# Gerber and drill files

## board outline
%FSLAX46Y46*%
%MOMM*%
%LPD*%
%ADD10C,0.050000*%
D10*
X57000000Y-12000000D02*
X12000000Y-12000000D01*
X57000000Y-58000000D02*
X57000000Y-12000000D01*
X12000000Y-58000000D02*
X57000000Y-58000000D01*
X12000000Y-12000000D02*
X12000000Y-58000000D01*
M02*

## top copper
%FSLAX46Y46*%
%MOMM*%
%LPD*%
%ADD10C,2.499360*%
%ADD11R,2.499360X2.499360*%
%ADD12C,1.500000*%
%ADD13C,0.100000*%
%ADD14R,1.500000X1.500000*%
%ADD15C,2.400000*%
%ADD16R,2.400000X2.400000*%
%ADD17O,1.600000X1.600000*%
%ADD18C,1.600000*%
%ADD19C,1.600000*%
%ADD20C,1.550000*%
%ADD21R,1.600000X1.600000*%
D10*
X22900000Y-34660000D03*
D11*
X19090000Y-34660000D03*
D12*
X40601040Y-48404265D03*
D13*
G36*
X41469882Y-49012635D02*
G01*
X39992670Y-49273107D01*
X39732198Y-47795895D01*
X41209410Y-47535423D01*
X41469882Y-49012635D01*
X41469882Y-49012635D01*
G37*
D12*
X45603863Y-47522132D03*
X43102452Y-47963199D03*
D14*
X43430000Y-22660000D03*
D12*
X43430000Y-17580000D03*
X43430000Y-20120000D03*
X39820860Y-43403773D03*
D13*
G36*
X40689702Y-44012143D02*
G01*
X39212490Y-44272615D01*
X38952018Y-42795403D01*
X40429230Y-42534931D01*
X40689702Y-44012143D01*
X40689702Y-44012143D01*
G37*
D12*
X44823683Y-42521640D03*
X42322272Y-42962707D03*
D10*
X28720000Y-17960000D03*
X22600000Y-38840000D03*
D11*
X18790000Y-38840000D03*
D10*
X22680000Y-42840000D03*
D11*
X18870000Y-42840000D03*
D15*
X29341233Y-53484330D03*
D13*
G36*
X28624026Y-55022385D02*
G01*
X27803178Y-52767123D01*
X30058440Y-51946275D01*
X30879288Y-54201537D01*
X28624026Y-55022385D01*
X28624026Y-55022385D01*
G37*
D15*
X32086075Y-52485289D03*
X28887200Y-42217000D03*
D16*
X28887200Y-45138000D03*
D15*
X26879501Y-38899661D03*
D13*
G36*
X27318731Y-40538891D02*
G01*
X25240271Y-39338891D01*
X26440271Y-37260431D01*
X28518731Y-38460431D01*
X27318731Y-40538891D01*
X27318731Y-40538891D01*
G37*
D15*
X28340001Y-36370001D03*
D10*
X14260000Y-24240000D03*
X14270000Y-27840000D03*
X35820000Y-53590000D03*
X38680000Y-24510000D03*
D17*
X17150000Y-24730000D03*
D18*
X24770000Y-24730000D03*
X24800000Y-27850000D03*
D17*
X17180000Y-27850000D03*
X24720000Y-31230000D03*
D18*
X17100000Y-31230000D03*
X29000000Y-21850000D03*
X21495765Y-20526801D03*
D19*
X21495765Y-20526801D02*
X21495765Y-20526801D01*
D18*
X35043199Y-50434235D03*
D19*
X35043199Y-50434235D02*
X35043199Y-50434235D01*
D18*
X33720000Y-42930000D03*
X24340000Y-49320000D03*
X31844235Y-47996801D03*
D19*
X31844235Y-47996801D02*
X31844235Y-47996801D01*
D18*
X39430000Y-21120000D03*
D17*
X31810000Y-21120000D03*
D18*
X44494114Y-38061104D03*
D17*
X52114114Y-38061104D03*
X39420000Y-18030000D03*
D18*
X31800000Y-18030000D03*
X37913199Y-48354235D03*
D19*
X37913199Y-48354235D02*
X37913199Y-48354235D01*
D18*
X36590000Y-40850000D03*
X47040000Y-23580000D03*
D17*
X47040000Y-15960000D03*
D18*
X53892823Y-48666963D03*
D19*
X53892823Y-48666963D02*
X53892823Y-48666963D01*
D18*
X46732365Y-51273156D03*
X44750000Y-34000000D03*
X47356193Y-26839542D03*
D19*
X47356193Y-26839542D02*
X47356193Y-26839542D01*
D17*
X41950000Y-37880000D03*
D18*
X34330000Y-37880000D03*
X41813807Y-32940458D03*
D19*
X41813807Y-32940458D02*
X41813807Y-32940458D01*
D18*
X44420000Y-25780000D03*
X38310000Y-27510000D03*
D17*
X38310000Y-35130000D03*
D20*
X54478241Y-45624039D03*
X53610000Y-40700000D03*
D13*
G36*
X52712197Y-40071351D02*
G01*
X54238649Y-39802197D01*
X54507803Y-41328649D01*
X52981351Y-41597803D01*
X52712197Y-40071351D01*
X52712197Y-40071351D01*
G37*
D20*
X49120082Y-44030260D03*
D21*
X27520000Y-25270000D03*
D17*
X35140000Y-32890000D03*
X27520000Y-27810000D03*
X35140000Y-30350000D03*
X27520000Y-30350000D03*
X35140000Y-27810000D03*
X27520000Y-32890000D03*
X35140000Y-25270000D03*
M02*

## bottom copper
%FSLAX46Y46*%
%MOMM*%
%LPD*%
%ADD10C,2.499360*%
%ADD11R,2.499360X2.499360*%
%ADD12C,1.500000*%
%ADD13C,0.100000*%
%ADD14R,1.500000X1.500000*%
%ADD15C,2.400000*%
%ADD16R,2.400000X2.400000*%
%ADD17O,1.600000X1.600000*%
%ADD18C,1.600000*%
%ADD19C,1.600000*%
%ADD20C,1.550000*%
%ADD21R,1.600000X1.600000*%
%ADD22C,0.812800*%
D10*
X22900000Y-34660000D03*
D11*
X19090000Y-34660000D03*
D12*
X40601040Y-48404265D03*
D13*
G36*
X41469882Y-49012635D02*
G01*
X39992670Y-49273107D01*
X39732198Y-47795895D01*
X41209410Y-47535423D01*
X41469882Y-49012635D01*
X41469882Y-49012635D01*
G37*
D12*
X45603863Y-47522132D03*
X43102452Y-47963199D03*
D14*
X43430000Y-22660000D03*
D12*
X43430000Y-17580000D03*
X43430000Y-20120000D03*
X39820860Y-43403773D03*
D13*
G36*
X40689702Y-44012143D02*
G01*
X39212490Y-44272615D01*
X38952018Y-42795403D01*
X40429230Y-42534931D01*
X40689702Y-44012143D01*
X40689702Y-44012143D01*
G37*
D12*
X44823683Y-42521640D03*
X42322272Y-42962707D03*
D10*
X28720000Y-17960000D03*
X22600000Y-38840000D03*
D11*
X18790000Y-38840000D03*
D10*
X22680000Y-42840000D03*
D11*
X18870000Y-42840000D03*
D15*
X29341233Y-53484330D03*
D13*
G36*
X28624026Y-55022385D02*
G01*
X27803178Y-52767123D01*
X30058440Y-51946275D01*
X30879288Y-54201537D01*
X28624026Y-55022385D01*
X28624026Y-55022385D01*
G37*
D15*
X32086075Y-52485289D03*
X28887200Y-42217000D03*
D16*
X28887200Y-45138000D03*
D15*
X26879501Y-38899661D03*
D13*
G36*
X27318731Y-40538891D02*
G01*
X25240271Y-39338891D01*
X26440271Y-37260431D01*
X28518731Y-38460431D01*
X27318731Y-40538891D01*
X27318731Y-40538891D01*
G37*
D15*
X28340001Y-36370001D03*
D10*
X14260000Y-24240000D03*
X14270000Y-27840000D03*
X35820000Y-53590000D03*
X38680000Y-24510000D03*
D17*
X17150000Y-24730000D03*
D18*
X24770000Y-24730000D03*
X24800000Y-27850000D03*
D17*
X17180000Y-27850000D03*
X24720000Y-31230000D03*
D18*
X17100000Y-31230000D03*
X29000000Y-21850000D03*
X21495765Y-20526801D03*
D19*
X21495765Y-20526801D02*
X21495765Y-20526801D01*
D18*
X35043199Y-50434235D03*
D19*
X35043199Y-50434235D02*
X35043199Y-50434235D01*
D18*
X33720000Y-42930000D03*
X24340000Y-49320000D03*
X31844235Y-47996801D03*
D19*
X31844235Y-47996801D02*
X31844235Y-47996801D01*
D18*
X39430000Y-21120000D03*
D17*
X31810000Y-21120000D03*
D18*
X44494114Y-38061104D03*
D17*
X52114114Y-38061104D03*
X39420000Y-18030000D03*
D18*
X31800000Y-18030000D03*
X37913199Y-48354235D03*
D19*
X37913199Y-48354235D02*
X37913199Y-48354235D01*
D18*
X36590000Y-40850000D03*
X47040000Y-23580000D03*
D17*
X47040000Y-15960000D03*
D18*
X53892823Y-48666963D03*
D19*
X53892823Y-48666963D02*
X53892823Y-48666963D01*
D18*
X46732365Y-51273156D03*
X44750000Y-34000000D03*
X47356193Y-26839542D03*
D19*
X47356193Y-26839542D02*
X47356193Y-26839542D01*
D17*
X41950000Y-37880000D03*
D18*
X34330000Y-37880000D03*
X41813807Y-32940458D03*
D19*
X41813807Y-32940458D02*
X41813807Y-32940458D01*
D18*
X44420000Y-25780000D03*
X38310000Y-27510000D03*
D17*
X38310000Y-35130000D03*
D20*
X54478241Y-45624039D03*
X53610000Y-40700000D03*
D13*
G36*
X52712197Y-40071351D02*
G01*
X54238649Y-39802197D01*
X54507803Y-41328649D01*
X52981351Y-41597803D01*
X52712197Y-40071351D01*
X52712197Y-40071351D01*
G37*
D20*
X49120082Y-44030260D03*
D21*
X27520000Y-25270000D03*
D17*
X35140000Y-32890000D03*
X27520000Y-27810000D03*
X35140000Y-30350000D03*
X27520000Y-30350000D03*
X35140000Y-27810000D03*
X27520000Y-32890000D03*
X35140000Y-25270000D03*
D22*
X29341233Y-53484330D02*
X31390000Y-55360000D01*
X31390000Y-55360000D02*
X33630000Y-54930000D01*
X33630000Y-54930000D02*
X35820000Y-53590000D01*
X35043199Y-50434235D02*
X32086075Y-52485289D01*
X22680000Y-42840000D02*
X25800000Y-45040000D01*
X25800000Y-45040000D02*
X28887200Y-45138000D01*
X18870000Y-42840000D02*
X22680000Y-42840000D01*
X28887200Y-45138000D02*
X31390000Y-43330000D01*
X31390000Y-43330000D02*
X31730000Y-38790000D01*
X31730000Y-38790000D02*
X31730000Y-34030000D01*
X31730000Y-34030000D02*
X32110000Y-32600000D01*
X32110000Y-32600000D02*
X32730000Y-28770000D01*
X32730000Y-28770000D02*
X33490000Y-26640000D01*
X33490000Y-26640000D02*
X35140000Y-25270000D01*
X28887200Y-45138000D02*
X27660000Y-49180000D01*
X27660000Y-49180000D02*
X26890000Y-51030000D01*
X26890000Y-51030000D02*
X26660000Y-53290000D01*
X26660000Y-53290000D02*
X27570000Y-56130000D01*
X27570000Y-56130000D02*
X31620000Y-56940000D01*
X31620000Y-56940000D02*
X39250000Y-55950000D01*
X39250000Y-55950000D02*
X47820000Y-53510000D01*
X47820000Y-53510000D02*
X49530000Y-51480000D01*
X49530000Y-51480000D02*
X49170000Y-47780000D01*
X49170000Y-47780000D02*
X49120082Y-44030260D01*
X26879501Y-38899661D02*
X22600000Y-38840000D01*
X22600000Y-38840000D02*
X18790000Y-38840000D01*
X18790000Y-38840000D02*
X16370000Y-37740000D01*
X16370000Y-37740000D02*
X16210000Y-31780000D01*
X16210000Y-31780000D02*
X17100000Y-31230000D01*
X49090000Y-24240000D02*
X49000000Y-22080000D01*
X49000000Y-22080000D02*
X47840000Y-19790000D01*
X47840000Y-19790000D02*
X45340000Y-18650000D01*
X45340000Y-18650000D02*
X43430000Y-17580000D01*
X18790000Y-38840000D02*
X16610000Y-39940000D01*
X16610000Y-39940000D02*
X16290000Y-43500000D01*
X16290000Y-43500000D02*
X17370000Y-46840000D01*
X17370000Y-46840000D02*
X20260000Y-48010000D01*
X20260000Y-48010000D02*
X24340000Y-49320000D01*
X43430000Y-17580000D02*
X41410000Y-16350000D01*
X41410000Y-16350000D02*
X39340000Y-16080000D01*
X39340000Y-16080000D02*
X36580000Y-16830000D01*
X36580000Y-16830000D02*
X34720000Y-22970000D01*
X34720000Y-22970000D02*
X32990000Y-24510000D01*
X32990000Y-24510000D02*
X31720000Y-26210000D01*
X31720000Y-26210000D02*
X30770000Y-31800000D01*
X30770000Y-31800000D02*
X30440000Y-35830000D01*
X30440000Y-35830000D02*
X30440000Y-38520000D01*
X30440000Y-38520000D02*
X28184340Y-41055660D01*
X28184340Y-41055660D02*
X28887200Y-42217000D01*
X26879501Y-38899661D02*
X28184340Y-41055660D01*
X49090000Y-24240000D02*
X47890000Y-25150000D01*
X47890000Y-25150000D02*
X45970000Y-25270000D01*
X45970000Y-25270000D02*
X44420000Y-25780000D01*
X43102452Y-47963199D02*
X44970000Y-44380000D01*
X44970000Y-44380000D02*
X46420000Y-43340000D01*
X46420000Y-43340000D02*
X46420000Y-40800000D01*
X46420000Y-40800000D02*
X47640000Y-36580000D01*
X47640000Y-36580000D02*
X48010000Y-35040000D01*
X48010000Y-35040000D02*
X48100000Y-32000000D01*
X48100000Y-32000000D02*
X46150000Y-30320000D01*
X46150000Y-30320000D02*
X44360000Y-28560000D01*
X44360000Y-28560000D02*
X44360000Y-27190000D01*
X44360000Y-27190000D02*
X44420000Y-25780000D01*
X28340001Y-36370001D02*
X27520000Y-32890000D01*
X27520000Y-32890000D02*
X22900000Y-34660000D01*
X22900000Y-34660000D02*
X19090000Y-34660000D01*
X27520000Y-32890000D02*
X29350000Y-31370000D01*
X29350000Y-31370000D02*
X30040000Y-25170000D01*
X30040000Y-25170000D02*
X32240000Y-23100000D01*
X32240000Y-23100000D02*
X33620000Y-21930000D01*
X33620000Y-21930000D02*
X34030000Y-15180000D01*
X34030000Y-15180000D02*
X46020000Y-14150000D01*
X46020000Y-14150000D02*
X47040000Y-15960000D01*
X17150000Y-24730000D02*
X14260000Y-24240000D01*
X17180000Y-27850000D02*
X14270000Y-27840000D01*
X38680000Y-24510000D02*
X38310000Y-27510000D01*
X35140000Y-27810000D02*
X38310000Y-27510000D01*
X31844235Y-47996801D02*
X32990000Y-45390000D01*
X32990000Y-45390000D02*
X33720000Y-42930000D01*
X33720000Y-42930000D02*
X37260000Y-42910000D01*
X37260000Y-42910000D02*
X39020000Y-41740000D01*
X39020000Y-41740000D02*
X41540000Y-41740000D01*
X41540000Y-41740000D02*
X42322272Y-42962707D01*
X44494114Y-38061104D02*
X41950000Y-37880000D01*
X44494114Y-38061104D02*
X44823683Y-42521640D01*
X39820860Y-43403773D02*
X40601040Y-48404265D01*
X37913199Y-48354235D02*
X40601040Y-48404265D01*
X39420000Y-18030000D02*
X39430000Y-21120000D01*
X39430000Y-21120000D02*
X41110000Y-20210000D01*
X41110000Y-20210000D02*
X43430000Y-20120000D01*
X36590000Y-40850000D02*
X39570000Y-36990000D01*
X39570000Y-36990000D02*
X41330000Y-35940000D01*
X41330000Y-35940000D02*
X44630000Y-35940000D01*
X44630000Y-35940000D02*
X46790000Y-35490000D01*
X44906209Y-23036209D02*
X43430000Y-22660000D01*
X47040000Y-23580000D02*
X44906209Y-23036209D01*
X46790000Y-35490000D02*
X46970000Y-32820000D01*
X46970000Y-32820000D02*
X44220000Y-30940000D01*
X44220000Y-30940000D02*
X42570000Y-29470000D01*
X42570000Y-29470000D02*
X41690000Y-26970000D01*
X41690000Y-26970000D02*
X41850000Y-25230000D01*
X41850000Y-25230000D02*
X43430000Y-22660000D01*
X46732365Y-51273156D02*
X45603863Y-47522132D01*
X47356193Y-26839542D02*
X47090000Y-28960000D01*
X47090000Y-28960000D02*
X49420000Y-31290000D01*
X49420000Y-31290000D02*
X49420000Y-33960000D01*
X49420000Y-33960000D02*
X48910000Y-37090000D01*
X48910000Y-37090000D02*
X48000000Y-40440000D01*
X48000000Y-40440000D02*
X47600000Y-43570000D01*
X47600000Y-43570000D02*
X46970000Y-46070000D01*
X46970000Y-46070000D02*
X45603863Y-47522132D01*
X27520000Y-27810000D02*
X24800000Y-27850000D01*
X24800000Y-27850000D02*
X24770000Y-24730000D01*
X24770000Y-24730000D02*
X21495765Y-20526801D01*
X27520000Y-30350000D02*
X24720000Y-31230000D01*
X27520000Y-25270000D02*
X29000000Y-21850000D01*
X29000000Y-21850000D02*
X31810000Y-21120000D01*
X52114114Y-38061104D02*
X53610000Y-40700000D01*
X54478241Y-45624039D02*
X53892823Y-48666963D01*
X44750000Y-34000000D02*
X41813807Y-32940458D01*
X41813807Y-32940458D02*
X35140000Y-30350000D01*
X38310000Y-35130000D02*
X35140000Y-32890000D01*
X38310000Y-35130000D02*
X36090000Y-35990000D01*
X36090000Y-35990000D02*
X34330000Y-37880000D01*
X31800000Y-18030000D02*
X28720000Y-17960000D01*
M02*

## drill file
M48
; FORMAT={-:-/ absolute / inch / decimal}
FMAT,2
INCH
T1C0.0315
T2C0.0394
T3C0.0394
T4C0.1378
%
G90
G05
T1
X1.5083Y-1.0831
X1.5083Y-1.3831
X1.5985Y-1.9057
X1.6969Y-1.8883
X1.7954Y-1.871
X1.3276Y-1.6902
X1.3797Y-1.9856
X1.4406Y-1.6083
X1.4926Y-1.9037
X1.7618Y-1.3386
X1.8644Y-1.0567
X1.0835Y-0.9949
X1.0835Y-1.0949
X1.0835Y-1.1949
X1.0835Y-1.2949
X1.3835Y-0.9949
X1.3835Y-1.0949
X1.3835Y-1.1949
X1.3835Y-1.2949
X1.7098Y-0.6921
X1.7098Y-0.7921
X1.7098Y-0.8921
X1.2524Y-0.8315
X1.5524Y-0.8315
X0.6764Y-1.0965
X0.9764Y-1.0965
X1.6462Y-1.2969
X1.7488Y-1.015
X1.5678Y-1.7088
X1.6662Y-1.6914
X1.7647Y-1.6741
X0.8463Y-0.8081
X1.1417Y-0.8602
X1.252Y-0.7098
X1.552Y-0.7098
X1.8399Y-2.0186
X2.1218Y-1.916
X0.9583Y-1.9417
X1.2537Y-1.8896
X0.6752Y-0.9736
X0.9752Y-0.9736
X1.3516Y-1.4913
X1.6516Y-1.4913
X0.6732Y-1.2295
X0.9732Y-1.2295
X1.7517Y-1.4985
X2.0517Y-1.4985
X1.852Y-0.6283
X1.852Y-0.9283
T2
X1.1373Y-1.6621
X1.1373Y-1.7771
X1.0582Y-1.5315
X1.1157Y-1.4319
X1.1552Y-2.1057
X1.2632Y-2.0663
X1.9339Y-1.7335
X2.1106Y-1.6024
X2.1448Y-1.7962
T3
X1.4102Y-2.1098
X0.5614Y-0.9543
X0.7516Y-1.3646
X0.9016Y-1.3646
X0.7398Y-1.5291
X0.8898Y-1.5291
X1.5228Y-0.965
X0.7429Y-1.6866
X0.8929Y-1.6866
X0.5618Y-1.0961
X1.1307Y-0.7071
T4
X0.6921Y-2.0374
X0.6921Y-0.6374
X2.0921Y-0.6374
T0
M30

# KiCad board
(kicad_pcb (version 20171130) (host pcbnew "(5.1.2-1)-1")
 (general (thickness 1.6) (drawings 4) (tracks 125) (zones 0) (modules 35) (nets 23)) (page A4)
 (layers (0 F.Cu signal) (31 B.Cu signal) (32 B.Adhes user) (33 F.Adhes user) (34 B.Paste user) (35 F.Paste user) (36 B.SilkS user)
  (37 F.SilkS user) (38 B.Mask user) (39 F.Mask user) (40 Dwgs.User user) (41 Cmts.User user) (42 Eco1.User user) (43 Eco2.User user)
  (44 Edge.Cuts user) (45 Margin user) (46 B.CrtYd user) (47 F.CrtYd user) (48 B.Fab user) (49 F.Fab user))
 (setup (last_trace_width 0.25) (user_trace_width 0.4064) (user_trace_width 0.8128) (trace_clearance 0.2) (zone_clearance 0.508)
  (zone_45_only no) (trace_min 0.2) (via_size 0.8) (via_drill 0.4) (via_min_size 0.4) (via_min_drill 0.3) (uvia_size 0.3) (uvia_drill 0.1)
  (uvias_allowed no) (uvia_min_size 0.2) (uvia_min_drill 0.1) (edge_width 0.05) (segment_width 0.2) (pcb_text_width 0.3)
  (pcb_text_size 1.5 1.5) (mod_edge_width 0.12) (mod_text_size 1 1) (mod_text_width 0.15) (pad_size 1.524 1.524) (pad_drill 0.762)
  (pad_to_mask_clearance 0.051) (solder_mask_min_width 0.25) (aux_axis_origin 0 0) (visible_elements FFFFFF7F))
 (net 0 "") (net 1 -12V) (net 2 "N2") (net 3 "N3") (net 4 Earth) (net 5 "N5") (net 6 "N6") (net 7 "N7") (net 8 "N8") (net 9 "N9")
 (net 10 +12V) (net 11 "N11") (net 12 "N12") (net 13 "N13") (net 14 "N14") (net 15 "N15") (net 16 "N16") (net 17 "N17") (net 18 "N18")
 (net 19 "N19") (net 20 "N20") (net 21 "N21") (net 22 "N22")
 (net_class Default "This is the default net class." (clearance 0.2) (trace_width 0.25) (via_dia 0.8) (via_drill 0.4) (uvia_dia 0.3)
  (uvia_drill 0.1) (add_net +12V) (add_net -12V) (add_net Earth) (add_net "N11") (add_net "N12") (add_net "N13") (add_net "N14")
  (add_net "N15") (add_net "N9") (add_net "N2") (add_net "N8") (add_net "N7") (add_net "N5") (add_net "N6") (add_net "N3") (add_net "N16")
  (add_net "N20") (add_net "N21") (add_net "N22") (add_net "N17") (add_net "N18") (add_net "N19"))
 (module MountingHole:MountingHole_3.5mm (layer F.Cu) (at 53.14 16.19)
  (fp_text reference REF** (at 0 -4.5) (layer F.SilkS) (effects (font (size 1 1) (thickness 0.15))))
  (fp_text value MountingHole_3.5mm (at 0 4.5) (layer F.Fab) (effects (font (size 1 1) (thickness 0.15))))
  (pad 1 np_thru_hole circle (at 0 0) (size 3.5 3.5) (drill 3.5) (layers *.Cu *.Mask)))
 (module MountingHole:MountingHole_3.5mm (layer F.Cu) (at 17.58 16.19)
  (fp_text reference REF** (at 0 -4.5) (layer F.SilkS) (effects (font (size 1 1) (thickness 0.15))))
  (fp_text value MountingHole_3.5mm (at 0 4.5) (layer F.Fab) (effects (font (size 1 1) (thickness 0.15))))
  (pad 1 np_thru_hole circle (at 0 0) (size 3.5 3.5) (drill 3.5) (layers *.Cu *.Mask)))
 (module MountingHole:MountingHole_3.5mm (layer F.Cu) (at 17.58 51.75)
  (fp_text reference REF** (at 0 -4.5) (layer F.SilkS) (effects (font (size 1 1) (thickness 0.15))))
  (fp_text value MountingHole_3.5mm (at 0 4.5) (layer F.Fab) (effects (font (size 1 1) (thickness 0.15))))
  (pad 1 np_thru_hole circle (at 0 0) (size 3.5 3.5) (drill 3.5) (layers *.Cu *.Mask)))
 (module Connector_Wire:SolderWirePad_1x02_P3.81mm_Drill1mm (layer F.Cu) (at 19.09 34.66)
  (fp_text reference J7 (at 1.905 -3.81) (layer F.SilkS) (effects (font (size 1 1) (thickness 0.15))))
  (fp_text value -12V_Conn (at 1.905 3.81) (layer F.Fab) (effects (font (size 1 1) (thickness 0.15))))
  (pad 2 thru_hole circle (at 3.81 0) (size 2.49936 2.49936) (drill 1.00076) (layers *.Cu *.Mask) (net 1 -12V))
  (pad 1 thru_hole rect (at 0 0) (size 2.49936 2.49936) (drill 1.00076) (layers *.Cu *.Mask) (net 1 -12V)))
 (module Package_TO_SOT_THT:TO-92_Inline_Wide (layer F.Cu) (at 40.60104 48.404265 10)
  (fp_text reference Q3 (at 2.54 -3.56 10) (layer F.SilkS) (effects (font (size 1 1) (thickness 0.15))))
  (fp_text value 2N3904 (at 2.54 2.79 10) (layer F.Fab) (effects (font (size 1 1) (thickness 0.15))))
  (pad 1 thru_hole rect (at 0 0 100) (size 1.5 1.5) (drill 0.8) (layers *.Cu *.Mask) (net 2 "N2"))
  (pad 3 thru_hole circle (at 5.08 0 100) (size 1.5 1.5) (drill 0.8) (layers *.Cu *.Mask) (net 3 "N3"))
  (pad 2 thru_hole circle (at 2.54 0 100) (size 1.5 1.5) (drill 0.8) (layers *.Cu *.Mask) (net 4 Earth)))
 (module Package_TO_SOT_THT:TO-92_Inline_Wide (layer F.Cu) (at 43.43 22.66 90)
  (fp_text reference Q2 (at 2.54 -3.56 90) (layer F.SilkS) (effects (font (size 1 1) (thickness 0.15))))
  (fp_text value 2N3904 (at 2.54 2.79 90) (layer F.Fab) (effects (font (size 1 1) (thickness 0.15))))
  (pad 1 thru_hole rect (at 0 0 180) (size 1.5 1.5) (drill 0.8) (layers *.Cu *.Mask) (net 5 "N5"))
  (pad 3 thru_hole circle (at 5.08 0 180) (size 1.5 1.5) (drill 0.8) (layers *.Cu *.Mask) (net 4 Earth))
  (pad 2 thru_hole circle (at 2.54 0 180) (size 1.5 1.5) (drill 0.8) (layers *.Cu *.Mask) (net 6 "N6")))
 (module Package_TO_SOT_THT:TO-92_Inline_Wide (layer F.Cu) (at 39.82086 43.403773 10)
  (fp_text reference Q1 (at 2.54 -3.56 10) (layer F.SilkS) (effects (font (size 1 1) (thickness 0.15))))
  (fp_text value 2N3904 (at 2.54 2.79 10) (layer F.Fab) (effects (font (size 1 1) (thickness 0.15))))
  (pad 1 thru_hole rect (at 0 0 100) (size 1.5 1.5) (drill 0.8) (layers *.Cu *.Mask) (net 2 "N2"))
  (pad 3 thru_hole circle (at 5.08 0 100) (size 1.5 1.5) (drill 0.8) (layers *.Cu *.Mask) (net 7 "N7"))
  (pad 2 thru_hole circle (at 2.54 0 100) (size 1.5 1.5) (drill 0.8) (layers *.Cu *.Mask) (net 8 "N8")))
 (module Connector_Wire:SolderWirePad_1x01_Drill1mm (layer F.Cu) (at 28.72 17.96)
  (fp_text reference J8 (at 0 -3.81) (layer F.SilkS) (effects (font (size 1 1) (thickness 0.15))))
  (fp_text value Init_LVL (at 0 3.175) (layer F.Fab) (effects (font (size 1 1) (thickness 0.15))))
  (pad 1 thru_hole circle (at 0 0) (size 2.49936 2.49936) (drill 1.00076) (layers *.Cu *.Mask) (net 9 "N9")))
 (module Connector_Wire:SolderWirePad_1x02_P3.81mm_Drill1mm (layer F.Cu) (at 18.79 38.84)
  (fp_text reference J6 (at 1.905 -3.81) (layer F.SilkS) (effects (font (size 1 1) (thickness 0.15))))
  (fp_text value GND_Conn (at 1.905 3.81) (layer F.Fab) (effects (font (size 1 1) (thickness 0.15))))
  (pad 2 thru_hole circle (at 3.81 0) (size 2.49936 2.49936) (drill 1.00076) (layers *.Cu *.Mask) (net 4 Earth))
  (pad 1 thru_hole rect (at 0 0) (size 2.49936 2.49936) (drill 1.00076) (layers *.Cu *.Mask) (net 4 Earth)))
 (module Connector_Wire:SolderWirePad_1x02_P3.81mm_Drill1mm (layer F.Cu) (at 18.87 42.84)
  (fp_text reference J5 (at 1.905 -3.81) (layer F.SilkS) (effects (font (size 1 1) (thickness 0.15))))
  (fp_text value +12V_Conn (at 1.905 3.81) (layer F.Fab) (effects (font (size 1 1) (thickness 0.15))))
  (pad 2 thru_hole circle (at 3.81 0) (size 2.49936 2.49936) (drill 1.00076) (layers *.Cu *.Mask) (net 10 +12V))
  (pad 1 thru_hole rect (at 0 0) (size 2.49936 2.49936) (drill 1.00076) (layers *.Cu *.Mask) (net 10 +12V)))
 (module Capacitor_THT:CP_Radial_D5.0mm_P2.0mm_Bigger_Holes (layer F.Cu) (at 31.29 53.64 20)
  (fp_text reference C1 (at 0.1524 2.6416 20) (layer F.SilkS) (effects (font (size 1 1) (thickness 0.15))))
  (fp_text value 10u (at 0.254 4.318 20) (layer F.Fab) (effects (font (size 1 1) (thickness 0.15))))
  (pad 1 thru_hole rect (at -1.778 -0.8128 20) (size 2.4 2.4) (drill 1) (layers *.Cu *.Mask) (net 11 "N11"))
  (pad 2 thru_hole circle (at 1.143 -0.8128 20) (size 2.4 2.4) (drill 1) (layers *.Cu *.Mask) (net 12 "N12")))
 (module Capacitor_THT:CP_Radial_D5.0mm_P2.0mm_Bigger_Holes (layer F.Cu) (at 29.7 43.36 90)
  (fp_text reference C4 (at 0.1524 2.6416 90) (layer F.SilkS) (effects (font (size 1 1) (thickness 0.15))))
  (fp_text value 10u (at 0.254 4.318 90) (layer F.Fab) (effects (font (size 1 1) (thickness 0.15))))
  (pad 2 thru_hole circle (at 1.143 -0.8128 90) (size 2.4 2.4) (drill 1) (layers *.Cu *.Mask) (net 4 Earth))
  (pad 1 thru_hole rect (at -1.778 -0.8128 90) (size 2.4 2.4) (drill 1) (layers *.Cu *.Mask) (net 10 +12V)))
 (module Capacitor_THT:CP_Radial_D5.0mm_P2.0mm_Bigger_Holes (layer F.Cu) (at 28.472406 37.766268 60)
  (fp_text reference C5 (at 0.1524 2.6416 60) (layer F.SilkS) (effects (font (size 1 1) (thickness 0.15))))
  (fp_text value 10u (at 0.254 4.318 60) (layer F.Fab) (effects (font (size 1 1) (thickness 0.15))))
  (pad 1 thru_hole rect (at -1.778 -0.8128 60) (size 2.4 2.4) (drill 1) (layers *.Cu *.Mask) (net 4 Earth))
  (pad 2 thru_hole circle (at 1.143 -0.8128 60) (size 2.4 2.4) (drill 1) (layers *.Cu *.Mask) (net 1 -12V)))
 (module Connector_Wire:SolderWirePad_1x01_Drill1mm (layer F.Cu) (at 14.26 24.24)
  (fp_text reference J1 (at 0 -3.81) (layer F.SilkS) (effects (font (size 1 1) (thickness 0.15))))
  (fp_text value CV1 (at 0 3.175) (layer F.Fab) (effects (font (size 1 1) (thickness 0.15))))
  (pad 1 thru_hole circle (at 0 0) (size 2.49936 2.49936) (drill 1.00076) (layers *.Cu *.Mask) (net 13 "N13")))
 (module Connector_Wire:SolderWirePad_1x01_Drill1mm (layer F.Cu) (at 14.27 27.84)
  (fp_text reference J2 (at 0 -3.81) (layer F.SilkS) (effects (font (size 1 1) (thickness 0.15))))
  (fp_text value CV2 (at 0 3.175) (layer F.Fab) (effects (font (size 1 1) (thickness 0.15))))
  (pad 1 thru_hole circle (at 0 0) (size 2.49936 2.49936) (drill 1.00076) (layers *.Cu *.Mask) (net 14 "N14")))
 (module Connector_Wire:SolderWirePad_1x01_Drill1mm (layer F.Cu) (at 35.82 53.59 10)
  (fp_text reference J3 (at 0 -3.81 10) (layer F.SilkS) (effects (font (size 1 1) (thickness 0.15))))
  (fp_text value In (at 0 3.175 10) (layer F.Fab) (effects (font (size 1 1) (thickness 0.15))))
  (pad 1 thru_hole circle (at 0 0 10) (size 2.49936 2.49936) (drill 1.00076) (layers *.Cu *.Mask) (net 11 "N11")))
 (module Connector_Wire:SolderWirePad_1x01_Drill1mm (layer F.Cu) (at 38.68 24.51)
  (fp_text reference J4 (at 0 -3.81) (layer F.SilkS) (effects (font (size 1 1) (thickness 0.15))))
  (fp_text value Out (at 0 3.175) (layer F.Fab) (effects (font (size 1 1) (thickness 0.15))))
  (pad 1 thru_hole circle (at 0 0) (size 2.49936 2.49936) (drill 1.00076) (layers *.Cu *.Mask) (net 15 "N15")))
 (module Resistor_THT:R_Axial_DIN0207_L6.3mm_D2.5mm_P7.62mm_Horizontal (layer F.Cu) (at 24.77 24.73 180)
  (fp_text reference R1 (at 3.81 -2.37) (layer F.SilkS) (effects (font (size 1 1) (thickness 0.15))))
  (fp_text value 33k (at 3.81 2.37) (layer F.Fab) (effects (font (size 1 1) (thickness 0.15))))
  (pad 2 thru_hole oval (at 7.62 0 180) (size 1.6 1.6) (drill 0.8) (layers *.Cu *.Mask) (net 13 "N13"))
  (pad 1 thru_hole circle (at 0 0 180) (size 1.6 1.6) (drill 0.8) (layers *.Cu *.Mask) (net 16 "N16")))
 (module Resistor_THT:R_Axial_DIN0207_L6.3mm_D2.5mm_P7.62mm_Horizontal (layer F.Cu) (at 24.8 27.85 180)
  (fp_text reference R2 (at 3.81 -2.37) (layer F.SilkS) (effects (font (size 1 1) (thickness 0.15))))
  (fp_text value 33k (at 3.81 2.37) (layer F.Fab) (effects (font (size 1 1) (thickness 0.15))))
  (pad 1 thru_hole circle (at 0 0 180) (size 1.6 1.6) (drill 0.8) (layers *.Cu *.Mask) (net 16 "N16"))
  (pad 2 thru_hole oval (at 7.62 0 180) (size 1.6 1.6) (drill 0.8) (layers *.Cu *.Mask) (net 14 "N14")))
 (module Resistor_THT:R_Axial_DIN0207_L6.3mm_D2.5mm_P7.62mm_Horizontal (layer F.Cu) (at 17.1 31.23)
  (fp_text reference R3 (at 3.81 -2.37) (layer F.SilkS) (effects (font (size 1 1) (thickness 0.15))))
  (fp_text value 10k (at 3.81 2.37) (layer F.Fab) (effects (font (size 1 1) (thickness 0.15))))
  (pad 2 thru_hole oval (at 7.62 0) (size 1.6 1.6) (drill 0.8) (layers *.Cu *.Mask) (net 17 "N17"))
  (pad 1 thru_hole circle (at 0 0) (size 1.6 1.6) (drill 0.8) (layers *.Cu *.Mask) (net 4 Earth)))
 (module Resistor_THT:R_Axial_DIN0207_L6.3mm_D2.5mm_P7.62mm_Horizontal (layer F.Cu) (at 29 21.85 170)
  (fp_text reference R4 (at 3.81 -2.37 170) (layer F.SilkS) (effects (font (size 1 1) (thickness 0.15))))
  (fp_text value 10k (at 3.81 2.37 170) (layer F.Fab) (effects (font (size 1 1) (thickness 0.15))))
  (pad 1 thru_hole circle (at 0 0 170) (size 1.6 1.6) (drill 0.8) (layers *.Cu *.Mask) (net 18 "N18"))
  (pad 2 thru_hole oval (at 7.62 0 170) (size 1.6 1.6) (drill 0.8) (layers *.Cu *.Mask) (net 16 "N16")))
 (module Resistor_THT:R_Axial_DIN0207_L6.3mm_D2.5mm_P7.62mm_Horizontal (layer F.Cu) (at 33.72 42.93 280)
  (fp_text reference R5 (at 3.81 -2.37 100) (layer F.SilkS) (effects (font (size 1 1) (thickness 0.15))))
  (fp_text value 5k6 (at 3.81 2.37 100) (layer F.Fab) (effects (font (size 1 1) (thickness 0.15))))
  (pad 2 thru_hole oval (at 7.62 0 280) (size 1.6 1.6) (drill 0.8) (layers *.Cu *.Mask) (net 12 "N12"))
  (pad 1 thru_hole circle (at 0 0 280) (size 1.6 1.6) (drill 0.8) (layers *.Cu *.Mask) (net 8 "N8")))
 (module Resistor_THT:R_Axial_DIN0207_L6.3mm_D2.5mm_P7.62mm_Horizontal (layer F.Cu) (at 24.34 49.32 10)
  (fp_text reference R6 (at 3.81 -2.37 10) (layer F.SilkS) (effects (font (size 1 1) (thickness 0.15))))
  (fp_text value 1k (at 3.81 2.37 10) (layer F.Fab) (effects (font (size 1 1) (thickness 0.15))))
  (pad 1 thru_hole circle (at 0 0 10) (size 1.6 1.6) (drill 0.8) (layers *.Cu *.Mask) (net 4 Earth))
  (pad 2 thru_hole oval (at 7.62 0 10) (size 1.6 1.6) (drill 0.8) (layers *.Cu *.Mask) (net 8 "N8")))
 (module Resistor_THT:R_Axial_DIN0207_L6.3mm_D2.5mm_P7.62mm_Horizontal (layer F.Cu) (at 39.43 21.12 180)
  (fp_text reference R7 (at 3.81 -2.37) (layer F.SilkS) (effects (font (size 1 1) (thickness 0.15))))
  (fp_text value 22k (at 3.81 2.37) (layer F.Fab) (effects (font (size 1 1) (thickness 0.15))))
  (pad 1 thru_hole circle (at 0 0 180) (size 1.6 1.6) (drill 0.8) (layers *.Cu *.Mask) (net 6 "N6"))
  (pad 2 thru_hole oval (at 7.62 0 180) (size 1.6 1.6) (drill 0.8) (layers *.Cu *.Mask) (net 18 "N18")))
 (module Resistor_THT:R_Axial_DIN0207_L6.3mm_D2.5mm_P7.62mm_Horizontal (layer F.Cu) (at 44.494114 38.061104)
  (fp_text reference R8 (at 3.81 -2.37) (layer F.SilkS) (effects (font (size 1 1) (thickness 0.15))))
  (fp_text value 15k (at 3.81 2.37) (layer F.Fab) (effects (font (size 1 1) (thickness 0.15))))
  (pad 1 thru_hole circle (at 0 0) (size 1.6 1.6) (drill 0.8) (layers *.Cu *.Mask) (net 7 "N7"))
  (pad 2 thru_hole oval (at 7.62 0) (size 1.6 1.6) (drill 0.8) (layers *.Cu *.Mask) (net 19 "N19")))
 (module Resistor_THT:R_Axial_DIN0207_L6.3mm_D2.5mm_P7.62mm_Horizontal (layer F.Cu) (at 31.8 18.03)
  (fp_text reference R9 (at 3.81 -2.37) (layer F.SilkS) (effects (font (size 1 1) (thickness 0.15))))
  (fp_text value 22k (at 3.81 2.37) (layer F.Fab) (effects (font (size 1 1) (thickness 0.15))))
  (pad 2 thru_hole oval (at 7.62 0) (size 1.6 1.6) (drill 0.8) (layers *.Cu *.Mask) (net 6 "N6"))
  (pad 1 thru_hole circle (at 0 0) (size 1.6 1.6) (drill 0.8) (layers *.Cu *.Mask) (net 9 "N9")))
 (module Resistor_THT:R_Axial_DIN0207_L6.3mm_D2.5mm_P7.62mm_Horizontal (layer F.Cu) (at 36.59 40.85 280)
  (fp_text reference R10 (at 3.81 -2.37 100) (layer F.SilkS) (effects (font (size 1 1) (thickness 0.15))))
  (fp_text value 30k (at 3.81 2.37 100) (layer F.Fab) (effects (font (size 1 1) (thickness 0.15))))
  (pad 2 thru_hole oval (at 7.62 0 280) (size 1.6 1.6) (drill 0.8) (layers *.Cu *.Mask) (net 2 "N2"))
  (pad 1 thru_hole circle (at 0 0 280) (size 1.6 1.6) (drill 0.8) (layers *.Cu *.Mask) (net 5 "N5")))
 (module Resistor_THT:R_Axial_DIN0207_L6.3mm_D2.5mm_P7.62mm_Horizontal (layer F.Cu) (at 47.04 23.58 90)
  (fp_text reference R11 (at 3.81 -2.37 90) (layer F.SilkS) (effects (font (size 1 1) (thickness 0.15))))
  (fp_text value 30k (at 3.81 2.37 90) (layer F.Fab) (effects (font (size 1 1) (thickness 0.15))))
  (pad 1 thru_hole circle (at 0 0 90) (size 1.6 1.6) (drill 0.8) (layers *.Cu *.Mask) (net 5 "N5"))
  (pad 2 thru_hole oval (at 7.62 0 90) (size 1.6 1.6) (drill 0.8) (layers *.Cu *.Mask) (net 1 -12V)))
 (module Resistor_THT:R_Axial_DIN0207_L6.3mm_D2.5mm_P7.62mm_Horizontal (layer F.Cu) (at 46.732365 51.273156 20)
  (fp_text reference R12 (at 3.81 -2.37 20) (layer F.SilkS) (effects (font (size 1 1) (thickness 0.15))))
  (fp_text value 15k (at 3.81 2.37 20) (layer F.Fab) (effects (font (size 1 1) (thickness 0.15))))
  (pad 2 thru_hole oval (at 7.62 0 20) (size 1.6 1.6) (drill 0.8) (layers *.Cu *.Mask) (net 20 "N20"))
  (pad 1 thru_hole circle (at 0 0 20) (size 1.6 1.6) (drill 0.8) (layers *.Cu *.Mask) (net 3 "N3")))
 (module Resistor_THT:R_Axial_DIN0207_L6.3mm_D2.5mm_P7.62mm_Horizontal (layer F.Cu) (at 44.75 34 70)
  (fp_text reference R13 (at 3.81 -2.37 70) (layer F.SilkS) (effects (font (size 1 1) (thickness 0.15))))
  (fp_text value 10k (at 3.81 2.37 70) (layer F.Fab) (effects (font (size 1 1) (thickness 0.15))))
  (pad 1 thru_hole circle (at 0 0 70) (size 1.6 1.6) (drill 0.8) (layers *.Cu *.Mask) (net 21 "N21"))
  (pad 2 thru_hole oval (at 7.62 0 70) (size 1.6 1.6) (drill 0.8) (layers *.Cu *.Mask) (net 3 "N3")))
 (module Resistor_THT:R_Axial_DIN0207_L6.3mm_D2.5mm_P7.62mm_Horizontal (layer F.Cu) (at 34.33 37.88)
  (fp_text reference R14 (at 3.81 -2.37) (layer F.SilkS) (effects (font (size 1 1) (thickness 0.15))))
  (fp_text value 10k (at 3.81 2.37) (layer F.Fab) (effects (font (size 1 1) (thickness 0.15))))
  (pad 2 thru_hole oval (at 7.62 0) (size 1.6 1.6) (drill 0.8) (layers *.Cu *.Mask) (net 7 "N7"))
  (pad 1 thru_hole circle (at 0 0) (size 1.6 1.6) (drill 0.8) (layers *.Cu *.Mask) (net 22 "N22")))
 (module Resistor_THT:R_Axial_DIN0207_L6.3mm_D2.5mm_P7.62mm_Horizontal (layer F.Cu) (at 44.42 25.78 250)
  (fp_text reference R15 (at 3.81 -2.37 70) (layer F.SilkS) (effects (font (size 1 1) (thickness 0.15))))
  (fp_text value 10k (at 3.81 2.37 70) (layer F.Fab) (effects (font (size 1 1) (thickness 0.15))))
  (pad 2 thru_hole oval (at 7.62 0 250) (size 1.6 1.6) (drill 0.8) (layers *.Cu *.Mask) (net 21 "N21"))
  (pad 1 thru_hole circle (at 0 0 250) (size 1.6 1.6) (drill 0.8) (layers *.Cu *.Mask) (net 4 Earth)))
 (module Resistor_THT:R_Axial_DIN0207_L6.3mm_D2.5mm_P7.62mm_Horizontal (layer F.Cu) (at 38.31 27.51 270)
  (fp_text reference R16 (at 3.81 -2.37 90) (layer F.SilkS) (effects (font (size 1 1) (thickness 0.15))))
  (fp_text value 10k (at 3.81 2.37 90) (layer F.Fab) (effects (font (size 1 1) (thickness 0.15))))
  (pad 1 thru_hole circle (at 0 0 270) (size 1.6 1.6) (drill 0.8) (layers *.Cu *.Mask) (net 15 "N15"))
  (pad 2 thru_hole oval (at 7.62 0 270) (size 1.6 1.6) (drill 0.8) (layers *.Cu *.Mask) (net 22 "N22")))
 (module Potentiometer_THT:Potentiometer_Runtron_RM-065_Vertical (layer F.Cu) (at 53.61 40.7 280)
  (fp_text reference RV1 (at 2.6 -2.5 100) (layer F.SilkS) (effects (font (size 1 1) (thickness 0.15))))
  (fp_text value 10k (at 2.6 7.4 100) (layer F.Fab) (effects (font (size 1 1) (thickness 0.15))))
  (pad 3 thru_hole circle (at 5 0 280) (size 1.55 1.55) (drill 1) (layers *.Cu *.Mask) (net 20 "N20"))
  (pad 1 thru_hole rect (at 0 0 280) (size 1.55 1.55) (drill 1) (layers *.Cu *.Mask) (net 19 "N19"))
  (pad 2 thru_hole circle (at 2.5 5 280) (size 1.55 1.55) (drill 1) (layers *.Cu *.Mask) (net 10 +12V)))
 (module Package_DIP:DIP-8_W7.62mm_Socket (layer F.Cu) (at 27.52 25.27)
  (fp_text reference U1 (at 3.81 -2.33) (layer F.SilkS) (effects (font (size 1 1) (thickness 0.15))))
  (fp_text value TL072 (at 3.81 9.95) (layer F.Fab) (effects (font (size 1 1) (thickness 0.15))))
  (pad 1 thru_hole rect (at 0 0) (size 1.6 1.6) (drill 0.8) (layers *.Cu *.Mask) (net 18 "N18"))
  (pad 5 thru_hole oval (at 7.62 7.62) (size 1.6 1.6) (drill 0.8) (layers *.Cu *.Mask) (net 22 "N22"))
  (pad 2 thru_hole oval (at 0 2.54) (size 1.6 1.6) (drill 0.8) (layers *.Cu *.Mask) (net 16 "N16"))
  (pad 6 thru_hole oval (at 7.62 5.08) (size 1.6 1.6) (drill 0.8) (layers *.Cu *.Mask) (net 21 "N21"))
  (pad 3 thru_hole oval (at 0 5.08) (size 1.6 1.6) (drill 0.8) (layers *.Cu *.Mask) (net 17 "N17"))
  (pad 7 thru_hole oval (at 7.62 2.54) (size 1.6 1.6) (drill 0.8) (layers *.Cu *.Mask) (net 15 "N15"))
  (pad 4 thru_hole oval (at 0 7.62) (size 1.6 1.6) (drill 0.8) (layers *.Cu *.Mask) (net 1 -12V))
  (pad 8 thru_hole oval (at 7.62 0) (size 1.6 1.6) (drill 0.8) (layers *.Cu *.Mask) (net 10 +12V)))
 (gr_line (start 57 12) (end 12 12) (layer Edge.Cuts) (width 0.05))
 (gr_line (start 57 58) (end 57 12) (layer Edge.Cuts) (width 0.05))
 (gr_line (start 12 58) (end 57 58) (layer Edge.Cuts) (width 0.05))
 (gr_line (start 12 12) (end 12 58) (layer Edge.Cuts) (width 0.05))
 (segment (start 29.341233 53.48433) (end 31.39 55.36) (width 0.8128) (layer B.Cu) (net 11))
 (segment (start 31.39 55.36) (end 33.63 54.93) (width 0.8128) (layer B.Cu) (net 11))
 (segment (start 33.63 54.93) (end 35.82 53.59) (width 0.8128) (layer B.Cu) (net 11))
 (segment (start 35.043199 50.434235) (end 32.086075 52.485289) (width 0.8128) (layer B.Cu) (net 12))
 (segment (start 22.68 42.84) (end 25.8 45.04) (width 0.8128) (layer B.Cu) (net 10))
 (segment (start 25.8 45.04) (end 28.8872 45.138) (width 0.8128) (layer B.Cu) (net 10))
 (segment (start 18.87 42.84) (end 22.68 42.84) (width 0.8128) (layer B.Cu) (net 10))
 (segment (start 28.8872 45.138) (end 31.39 43.33) (width 0.8128) (layer B.Cu) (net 10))
 (segment (start 31.39 43.33) (end 31.73 38.79) (width 0.8128) (layer B.Cu) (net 10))
 (segment (start 31.73 38.79) (end 31.73 34.03) (width 0.8128) (layer B.Cu) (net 10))
 (segment (start 31.73 34.03) (end 32.11 32.6) (width 0.8128) (layer B.Cu) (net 10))
 (segment (start 32.11 32.6) (end 32.73 28.77) (width 0.8128) (layer B.Cu) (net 10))
 (segment (start 32.73 28.77) (end 33.49 26.64) (width 0.8128) (layer B.Cu) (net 10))
 (segment (start 33.49 26.64) (end 35.14 25.27) (width 0.8128) (layer B.Cu) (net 10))
 (segment (start 28.8872 45.138) (end 27.66 49.18) (width 0.8128) (layer B.Cu) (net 10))
 (segment (start 27.66 49.18) (end 26.89 51.03) (width 0.8128) (layer B.Cu) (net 10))
 (segment (start 26.89 51.03) (end 26.66 53.29) (width 0.8128) (layer B.Cu) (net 10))
 (segment (start 26.66 53.29) (end 27.57 56.13) (width 0.8128) (layer B.Cu) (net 10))
 (segment (start 27.57 56.13) (end 31.62 56.94) (width 0.8128) (layer B.Cu) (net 10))
 (segment (start 31.62 56.94) (end 39.25 55.95) (width 0.8128) (layer B.Cu) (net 10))
 (segment (start 39.25 55.95) (end 47.82 53.51) (width 0.8128) (layer B.Cu) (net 10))
 (segment (start 47.82 53.51) (end 49.53 51.48) (width 0.8128) (layer B.Cu) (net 10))
 (segment (start 49.53 51.48) (end 49.17 47.78) (width 0.8128) (layer B.Cu) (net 10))
 (segment (start 49.17 47.78) (end 49.120082 44.03026) (width 0.8128) (layer B.Cu) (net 10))
 (segment (start 26.879501 38.899661) (end 22.6 38.84) (width 0.8128) (layer B.Cu) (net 4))
 (segment (start 22.6 38.84) (end 18.79 38.84) (width 0.8128) (layer B.Cu) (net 4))
 (segment (start 18.79 38.84) (end 16.37 37.74) (width 0.8128) (layer B.Cu) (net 4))
 (segment (start 16.37 37.74) (end 16.21 31.78) (width 0.8128) (layer B.Cu) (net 4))
 (segment (start 16.21 31.78) (end 17.1 31.23) (width 0.8128) (layer B.Cu) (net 4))
 (segment (start 49.09 24.24) (end 49 22.08) (width 0.8128) (layer B.Cu) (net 4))
 (segment (start 49 22.08) (end 47.84 19.79) (width 0.8128) (layer B.Cu) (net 4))
 (segment (start 47.84 19.79) (end 45.34 18.65) (width 0.8128) (layer B.Cu) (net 4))
 (segment (start 45.34 18.65) (end 43.43 17.58) (width 0.8128) (layer B.Cu) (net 4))
 (segment (start 18.79 38.84) (end 16.61 39.94) (width 0.8128) (layer B.Cu) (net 4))
 (segment (start 16.61 39.94) (end 16.29 43.5) (width 0.8128) (layer B.Cu) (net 4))
 (segment (start 16.29 43.5) (end 17.37 46.84) (width 0.8128) (layer B.Cu) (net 4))
 (segment (start 17.37 46.84) (end 20.26 48.01) (width 0.8128) (layer B.Cu) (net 4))
 (segment (start 20.26 48.01) (end 24.34 49.32) (width 0.8128) (layer B.Cu) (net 4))
 (segment (start 43.43 17.58) (end 41.41 16.35) (width 0.8128) (layer B.Cu) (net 4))
 (segment (start 41.41 16.35) (end 39.34 16.08) (width 0.8128) (layer B.Cu) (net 4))
 (segment (start 39.34 16.08) (end 36.58 16.83) (width 0.8128) (layer B.Cu) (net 4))
 (segment (start 36.58 16.83) (end 34.72 22.97) (width 0.8128) (layer B.Cu) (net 4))
 (segment (start 34.72 22.97) (end 32.99 24.51) (width 0.8128) (layer B.Cu) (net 4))
 (segment (start 32.99 24.51) (end 31.72 26.21) (width 0.8128) (layer B.Cu) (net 4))
 (segment (start 31.72 26.21) (end 30.77 31.8) (width 0.8128) (layer B.Cu) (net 4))
 (segment (start 30.77 31.8) (end 30.44 35.83) (width 0.8128) (layer B.Cu) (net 4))
 (segment (start 30.44 35.83) (end 30.44 38.52) (width 0.8128) (layer B.Cu) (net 4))
 (segment (start 30.44 38.52) (end 28.18434 41.05566) (width 0.8128) (layer B.Cu) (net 4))
 (segment (start 28.18434 41.05566) (end 28.8872 42.217) (width 0.8128) (layer B.Cu) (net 4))
 (segment (start 26.879501 38.899661) (end 28.18434 41.05566) (width 0.8128) (layer B.Cu) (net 4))
 (segment (start 49.09 24.24) (end 47.89 25.15) (width 0.8128) (layer B.Cu) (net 4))
 (segment (start 47.89 25.15) (end 45.97 25.27) (width 0.8128) (layer B.Cu) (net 4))
 (segment (start 45.97 25.27) (end 44.42 25.78) (width 0.8128) (layer B.Cu) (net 4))
 (segment (start 43.102452 47.963199) (end 44.97 44.38) (width 0.8128) (layer B.Cu) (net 4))
 (segment (start 44.97 44.38) (end 46.42 43.34) (width 0.8128) (layer B.Cu) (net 4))
 (segment (start 46.42 43.34) (end 46.42 40.8) (width 0.8128) (layer B.Cu) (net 4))
 (segment (start 46.42 40.8) (end 47.64 36.58) (width 0.8128) (layer B.Cu) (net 4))
 (segment (start 47.64 36.58) (end 48.01 35.04) (width 0.8128) (layer B.Cu) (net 4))
 (segment (start 48.01 35.04) (end 48.1 32) (width 0.8128) (layer B.Cu) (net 4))
 (segment (start 48.1 32) (end 46.15 30.32) (width 0.8128) (layer B.Cu) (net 4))
 (segment (start 46.15 30.32) (end 44.36 28.56) (width 0.8128) (layer B.Cu) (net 4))
 (segment (start 44.36 28.56) (end 44.36 27.19) (width 0.8128) (layer B.Cu) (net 4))
 (segment (start 44.36 27.19) (end 44.42 25.78) (width 0.8128) (layer B.Cu) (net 4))
 (segment (start 28.340001 36.370001) (end 27.52 32.89) (width 0.8128) (layer B.Cu) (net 1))
 (segment (start 27.52 32.89) (end 22.9 34.66) (width 0.8128) (layer B.Cu) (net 1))
 (segment (start 22.9 34.66) (end 19.09 34.66) (width 0.8128) (layer B.Cu) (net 1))
 (segment (start 27.52 32.89) (end 29.35 31.37) (width 0.8128) (layer B.Cu) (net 1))
 (segment (start 29.35 31.37) (end 30.04 25.17) (width 0.8128) (layer B.Cu) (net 1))
 (segment (start 30.04 25.17) (end 32.24 23.1) (width 0.8128) (layer B.Cu) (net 1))
 (segment (start 32.24 23.1) (end 33.62 21.93) (width 0.8128) (layer B.Cu) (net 1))
 (segment (start 33.62 21.93) (end 34.03 15.18) (width 0.8128) (layer B.Cu) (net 1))
 (segment (start 34.03 15.18) (end 46.02 14.15) (width 0.8128) (layer B.Cu) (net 1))
 (segment (start 46.02 14.15) (end 47.04 15.96) (width 0.8128) (layer B.Cu) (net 1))
 (segment (start 17.15 24.73) (end 14.26 24.24) (width 0.8128) (layer B.Cu) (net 13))
 (segment (start 17.18 27.85) (end 14.27 27.84) (width 0.8128) (layer B.Cu) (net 14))
 (segment (start 38.68 24.51) (end 38.31 27.51) (width 0.8128) (layer B.Cu) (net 15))
 (segment (start 35.14 27.81) (end 38.31 27.51) (width 0.8128) (layer B.Cu) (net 15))
 (segment (start 31.844235 47.996801) (end 32.99 45.39) (width 0.8128) (layer B.Cu) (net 8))
 (segment (start 32.99 45.39) (end 33.72 42.93) (width 0.8128) (layer B.Cu) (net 8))
 (segment (start 33.72 42.93) (end 37.26 42.91) (width 0.8128) (layer B.Cu) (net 8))
 (segment (start 37.26 42.91) (end 39.02 41.74) (width 0.8128) (layer B.Cu) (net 8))
 (segment (start 39.02 41.74) (end 41.54 41.74) (width 0.8128) (layer B.Cu) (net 8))
 (segment (start 41.54 41.74) (end 42.322272 42.962707) (width 0.8128) (layer B.Cu) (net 8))
 (segment (start 44.494114 38.061104) (end 41.95 37.88) (width 0.8128) (layer B.Cu) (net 7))
 (segment (start 44.494114 38.061104) (end 44.823683 42.52164) (width 0.8128) (layer B.Cu) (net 7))
 (segment (start 39.82086 43.403773) (end 40.60104 48.404265) (width 0.8128) (layer B.Cu) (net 2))
 (segment (start 37.913199 48.354235) (end 40.60104 48.404265) (width 0.8128) (layer B.Cu) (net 2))
 (segment (start 39.42 18.03) (end 39.43 21.12) (width 0.8128) (layer B.Cu) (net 6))
 (segment (start 39.43 21.12) (end 41.11 20.21) (width 0.8128) (layer B.Cu) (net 6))
 (segment (start 41.11 20.21) (end 43.43 20.12) (width 0.8128) (layer B.Cu) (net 6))
 (segment (start 36.59 40.85) (end 39.57 36.99) (width 0.8128) (layer B.Cu) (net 5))
 (segment (start 39.57 36.99) (end 41.33 35.94) (width 0.8128) (layer B.Cu) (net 5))
 (segment (start 41.33 35.94) (end 44.63 35.94) (width 0.8128) (layer B.Cu) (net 5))
 (segment (start 44.63 35.94) (end 46.79 35.49) (width 0.8128) (layer B.Cu) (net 5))
 (segment (start 44.906209 23.036209) (end 43.43 22.66) (width 0.8128) (layer B.Cu) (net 5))
 (segment (start 47.04 23.58) (end 44.906209 23.036209) (width 0.8128) (layer B.Cu) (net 5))
 (segment (start 46.79 35.49) (end 46.97 32.82) (width 0.8128) (layer B.Cu) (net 5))
 (segment (start 46.97 32.82) (end 44.22 30.94) (width 0.8128) (layer B.Cu) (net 5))
 (segment (start 44.22 30.94) (end 42.57 29.47) (width 0.8128) (layer B.Cu) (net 5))
 (segment (start 42.57 29.47) (end 41.69 26.97) (width 0.8128) (layer B.Cu) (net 5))
 (segment (start 41.69 26.97) (end 41.85 25.23) (width 0.8128) (layer B.Cu) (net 5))
 (segment (start 41.85 25.23) (end 43.43 22.66) (width 0.8128) (layer B.Cu) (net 5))
 (segment (start 46.732365 51.273156) (end 45.603863 47.522132) (width 0.8128) (layer B.Cu) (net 3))
 (segment (start 47.356193 26.839542) (end 47.09 28.96) (width 0.8128) (layer B.Cu) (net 3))
 (segment (start 47.09 28.96) (end 49.42 31.29) (width 0.8128) (layer B.Cu) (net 3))
 (segment (start 49.42 31.29) (end 49.42 33.96) (width 0.8128) (layer B.Cu) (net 3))
 (segment (start 49.42 33.96) (end 48.91 37.09) (width 0.8128) (layer B.Cu) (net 3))
 (segment (start 48.91 37.09) (end 48 40.44) (width 0.8128) (layer B.Cu) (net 3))
 (segment (start 48 40.44) (end 47.6 43.57) (width 0.8128) (layer B.Cu) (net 3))
 (segment (start 47.6 43.57) (end 46.97 46.07) (width 0.8128) (layer B.Cu) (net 3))
 (segment (start 46.97 46.07) (end 45.603863 47.522132) (width 0.8128) (layer B.Cu) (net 3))
 (segment (start 27.52 27.81) (end 24.8 27.85) (width 0.8128) (layer B.Cu) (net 16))
 (segment (start 24.8 27.85) (end 24.77 24.73) (width 0.8128) (layer B.Cu) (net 16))
 (segment (start 24.77 24.73) (end 21.495765 20.526801) (width 0.8128) (layer B.Cu) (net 16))
 (segment (start 27.52 30.35) (end 24.72 31.23) (width 0.8128) (layer B.Cu) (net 17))
 (segment (start 27.52 25.27) (end 29 21.85) (width 0.8128) (layer B.Cu) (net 18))
 (segment (start 29 21.85) (end 31.81 21.12) (width 0.8128) (layer B.Cu) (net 18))
 (segment (start 52.114114 38.061104) (end 53.61 40.7) (width 0.8128) (layer B.Cu) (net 19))
 (segment (start 54.478241 45.624039) (end 53.892823 48.666963) (width 0.8128) (layer B.Cu) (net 20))
 (segment (start 44.75 34) (end 41.813807 32.940458) (width 0.8128) (layer B.Cu) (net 21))
 (segment (start 41.813807 32.940458) (end 35.14 30.35) (width 0.8128) (layer B.Cu) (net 21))
 (segment (start 38.31 35.13) (end 35.14 32.89) (width 0.8128) (layer B.Cu) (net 22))
 (segment (start 38.31 35.13) (end 36.09 35.99) (width 0.8128) (layer B.Cu) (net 22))
 (segment (start 36.09 35.99) (end 34.33 37.88) (width 0.8128) (layer B.Cu) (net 22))
 (segment (start 31.8 18.03) (end 28.72 17.96) (width 0.8128) (layer B.Cu) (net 9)))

